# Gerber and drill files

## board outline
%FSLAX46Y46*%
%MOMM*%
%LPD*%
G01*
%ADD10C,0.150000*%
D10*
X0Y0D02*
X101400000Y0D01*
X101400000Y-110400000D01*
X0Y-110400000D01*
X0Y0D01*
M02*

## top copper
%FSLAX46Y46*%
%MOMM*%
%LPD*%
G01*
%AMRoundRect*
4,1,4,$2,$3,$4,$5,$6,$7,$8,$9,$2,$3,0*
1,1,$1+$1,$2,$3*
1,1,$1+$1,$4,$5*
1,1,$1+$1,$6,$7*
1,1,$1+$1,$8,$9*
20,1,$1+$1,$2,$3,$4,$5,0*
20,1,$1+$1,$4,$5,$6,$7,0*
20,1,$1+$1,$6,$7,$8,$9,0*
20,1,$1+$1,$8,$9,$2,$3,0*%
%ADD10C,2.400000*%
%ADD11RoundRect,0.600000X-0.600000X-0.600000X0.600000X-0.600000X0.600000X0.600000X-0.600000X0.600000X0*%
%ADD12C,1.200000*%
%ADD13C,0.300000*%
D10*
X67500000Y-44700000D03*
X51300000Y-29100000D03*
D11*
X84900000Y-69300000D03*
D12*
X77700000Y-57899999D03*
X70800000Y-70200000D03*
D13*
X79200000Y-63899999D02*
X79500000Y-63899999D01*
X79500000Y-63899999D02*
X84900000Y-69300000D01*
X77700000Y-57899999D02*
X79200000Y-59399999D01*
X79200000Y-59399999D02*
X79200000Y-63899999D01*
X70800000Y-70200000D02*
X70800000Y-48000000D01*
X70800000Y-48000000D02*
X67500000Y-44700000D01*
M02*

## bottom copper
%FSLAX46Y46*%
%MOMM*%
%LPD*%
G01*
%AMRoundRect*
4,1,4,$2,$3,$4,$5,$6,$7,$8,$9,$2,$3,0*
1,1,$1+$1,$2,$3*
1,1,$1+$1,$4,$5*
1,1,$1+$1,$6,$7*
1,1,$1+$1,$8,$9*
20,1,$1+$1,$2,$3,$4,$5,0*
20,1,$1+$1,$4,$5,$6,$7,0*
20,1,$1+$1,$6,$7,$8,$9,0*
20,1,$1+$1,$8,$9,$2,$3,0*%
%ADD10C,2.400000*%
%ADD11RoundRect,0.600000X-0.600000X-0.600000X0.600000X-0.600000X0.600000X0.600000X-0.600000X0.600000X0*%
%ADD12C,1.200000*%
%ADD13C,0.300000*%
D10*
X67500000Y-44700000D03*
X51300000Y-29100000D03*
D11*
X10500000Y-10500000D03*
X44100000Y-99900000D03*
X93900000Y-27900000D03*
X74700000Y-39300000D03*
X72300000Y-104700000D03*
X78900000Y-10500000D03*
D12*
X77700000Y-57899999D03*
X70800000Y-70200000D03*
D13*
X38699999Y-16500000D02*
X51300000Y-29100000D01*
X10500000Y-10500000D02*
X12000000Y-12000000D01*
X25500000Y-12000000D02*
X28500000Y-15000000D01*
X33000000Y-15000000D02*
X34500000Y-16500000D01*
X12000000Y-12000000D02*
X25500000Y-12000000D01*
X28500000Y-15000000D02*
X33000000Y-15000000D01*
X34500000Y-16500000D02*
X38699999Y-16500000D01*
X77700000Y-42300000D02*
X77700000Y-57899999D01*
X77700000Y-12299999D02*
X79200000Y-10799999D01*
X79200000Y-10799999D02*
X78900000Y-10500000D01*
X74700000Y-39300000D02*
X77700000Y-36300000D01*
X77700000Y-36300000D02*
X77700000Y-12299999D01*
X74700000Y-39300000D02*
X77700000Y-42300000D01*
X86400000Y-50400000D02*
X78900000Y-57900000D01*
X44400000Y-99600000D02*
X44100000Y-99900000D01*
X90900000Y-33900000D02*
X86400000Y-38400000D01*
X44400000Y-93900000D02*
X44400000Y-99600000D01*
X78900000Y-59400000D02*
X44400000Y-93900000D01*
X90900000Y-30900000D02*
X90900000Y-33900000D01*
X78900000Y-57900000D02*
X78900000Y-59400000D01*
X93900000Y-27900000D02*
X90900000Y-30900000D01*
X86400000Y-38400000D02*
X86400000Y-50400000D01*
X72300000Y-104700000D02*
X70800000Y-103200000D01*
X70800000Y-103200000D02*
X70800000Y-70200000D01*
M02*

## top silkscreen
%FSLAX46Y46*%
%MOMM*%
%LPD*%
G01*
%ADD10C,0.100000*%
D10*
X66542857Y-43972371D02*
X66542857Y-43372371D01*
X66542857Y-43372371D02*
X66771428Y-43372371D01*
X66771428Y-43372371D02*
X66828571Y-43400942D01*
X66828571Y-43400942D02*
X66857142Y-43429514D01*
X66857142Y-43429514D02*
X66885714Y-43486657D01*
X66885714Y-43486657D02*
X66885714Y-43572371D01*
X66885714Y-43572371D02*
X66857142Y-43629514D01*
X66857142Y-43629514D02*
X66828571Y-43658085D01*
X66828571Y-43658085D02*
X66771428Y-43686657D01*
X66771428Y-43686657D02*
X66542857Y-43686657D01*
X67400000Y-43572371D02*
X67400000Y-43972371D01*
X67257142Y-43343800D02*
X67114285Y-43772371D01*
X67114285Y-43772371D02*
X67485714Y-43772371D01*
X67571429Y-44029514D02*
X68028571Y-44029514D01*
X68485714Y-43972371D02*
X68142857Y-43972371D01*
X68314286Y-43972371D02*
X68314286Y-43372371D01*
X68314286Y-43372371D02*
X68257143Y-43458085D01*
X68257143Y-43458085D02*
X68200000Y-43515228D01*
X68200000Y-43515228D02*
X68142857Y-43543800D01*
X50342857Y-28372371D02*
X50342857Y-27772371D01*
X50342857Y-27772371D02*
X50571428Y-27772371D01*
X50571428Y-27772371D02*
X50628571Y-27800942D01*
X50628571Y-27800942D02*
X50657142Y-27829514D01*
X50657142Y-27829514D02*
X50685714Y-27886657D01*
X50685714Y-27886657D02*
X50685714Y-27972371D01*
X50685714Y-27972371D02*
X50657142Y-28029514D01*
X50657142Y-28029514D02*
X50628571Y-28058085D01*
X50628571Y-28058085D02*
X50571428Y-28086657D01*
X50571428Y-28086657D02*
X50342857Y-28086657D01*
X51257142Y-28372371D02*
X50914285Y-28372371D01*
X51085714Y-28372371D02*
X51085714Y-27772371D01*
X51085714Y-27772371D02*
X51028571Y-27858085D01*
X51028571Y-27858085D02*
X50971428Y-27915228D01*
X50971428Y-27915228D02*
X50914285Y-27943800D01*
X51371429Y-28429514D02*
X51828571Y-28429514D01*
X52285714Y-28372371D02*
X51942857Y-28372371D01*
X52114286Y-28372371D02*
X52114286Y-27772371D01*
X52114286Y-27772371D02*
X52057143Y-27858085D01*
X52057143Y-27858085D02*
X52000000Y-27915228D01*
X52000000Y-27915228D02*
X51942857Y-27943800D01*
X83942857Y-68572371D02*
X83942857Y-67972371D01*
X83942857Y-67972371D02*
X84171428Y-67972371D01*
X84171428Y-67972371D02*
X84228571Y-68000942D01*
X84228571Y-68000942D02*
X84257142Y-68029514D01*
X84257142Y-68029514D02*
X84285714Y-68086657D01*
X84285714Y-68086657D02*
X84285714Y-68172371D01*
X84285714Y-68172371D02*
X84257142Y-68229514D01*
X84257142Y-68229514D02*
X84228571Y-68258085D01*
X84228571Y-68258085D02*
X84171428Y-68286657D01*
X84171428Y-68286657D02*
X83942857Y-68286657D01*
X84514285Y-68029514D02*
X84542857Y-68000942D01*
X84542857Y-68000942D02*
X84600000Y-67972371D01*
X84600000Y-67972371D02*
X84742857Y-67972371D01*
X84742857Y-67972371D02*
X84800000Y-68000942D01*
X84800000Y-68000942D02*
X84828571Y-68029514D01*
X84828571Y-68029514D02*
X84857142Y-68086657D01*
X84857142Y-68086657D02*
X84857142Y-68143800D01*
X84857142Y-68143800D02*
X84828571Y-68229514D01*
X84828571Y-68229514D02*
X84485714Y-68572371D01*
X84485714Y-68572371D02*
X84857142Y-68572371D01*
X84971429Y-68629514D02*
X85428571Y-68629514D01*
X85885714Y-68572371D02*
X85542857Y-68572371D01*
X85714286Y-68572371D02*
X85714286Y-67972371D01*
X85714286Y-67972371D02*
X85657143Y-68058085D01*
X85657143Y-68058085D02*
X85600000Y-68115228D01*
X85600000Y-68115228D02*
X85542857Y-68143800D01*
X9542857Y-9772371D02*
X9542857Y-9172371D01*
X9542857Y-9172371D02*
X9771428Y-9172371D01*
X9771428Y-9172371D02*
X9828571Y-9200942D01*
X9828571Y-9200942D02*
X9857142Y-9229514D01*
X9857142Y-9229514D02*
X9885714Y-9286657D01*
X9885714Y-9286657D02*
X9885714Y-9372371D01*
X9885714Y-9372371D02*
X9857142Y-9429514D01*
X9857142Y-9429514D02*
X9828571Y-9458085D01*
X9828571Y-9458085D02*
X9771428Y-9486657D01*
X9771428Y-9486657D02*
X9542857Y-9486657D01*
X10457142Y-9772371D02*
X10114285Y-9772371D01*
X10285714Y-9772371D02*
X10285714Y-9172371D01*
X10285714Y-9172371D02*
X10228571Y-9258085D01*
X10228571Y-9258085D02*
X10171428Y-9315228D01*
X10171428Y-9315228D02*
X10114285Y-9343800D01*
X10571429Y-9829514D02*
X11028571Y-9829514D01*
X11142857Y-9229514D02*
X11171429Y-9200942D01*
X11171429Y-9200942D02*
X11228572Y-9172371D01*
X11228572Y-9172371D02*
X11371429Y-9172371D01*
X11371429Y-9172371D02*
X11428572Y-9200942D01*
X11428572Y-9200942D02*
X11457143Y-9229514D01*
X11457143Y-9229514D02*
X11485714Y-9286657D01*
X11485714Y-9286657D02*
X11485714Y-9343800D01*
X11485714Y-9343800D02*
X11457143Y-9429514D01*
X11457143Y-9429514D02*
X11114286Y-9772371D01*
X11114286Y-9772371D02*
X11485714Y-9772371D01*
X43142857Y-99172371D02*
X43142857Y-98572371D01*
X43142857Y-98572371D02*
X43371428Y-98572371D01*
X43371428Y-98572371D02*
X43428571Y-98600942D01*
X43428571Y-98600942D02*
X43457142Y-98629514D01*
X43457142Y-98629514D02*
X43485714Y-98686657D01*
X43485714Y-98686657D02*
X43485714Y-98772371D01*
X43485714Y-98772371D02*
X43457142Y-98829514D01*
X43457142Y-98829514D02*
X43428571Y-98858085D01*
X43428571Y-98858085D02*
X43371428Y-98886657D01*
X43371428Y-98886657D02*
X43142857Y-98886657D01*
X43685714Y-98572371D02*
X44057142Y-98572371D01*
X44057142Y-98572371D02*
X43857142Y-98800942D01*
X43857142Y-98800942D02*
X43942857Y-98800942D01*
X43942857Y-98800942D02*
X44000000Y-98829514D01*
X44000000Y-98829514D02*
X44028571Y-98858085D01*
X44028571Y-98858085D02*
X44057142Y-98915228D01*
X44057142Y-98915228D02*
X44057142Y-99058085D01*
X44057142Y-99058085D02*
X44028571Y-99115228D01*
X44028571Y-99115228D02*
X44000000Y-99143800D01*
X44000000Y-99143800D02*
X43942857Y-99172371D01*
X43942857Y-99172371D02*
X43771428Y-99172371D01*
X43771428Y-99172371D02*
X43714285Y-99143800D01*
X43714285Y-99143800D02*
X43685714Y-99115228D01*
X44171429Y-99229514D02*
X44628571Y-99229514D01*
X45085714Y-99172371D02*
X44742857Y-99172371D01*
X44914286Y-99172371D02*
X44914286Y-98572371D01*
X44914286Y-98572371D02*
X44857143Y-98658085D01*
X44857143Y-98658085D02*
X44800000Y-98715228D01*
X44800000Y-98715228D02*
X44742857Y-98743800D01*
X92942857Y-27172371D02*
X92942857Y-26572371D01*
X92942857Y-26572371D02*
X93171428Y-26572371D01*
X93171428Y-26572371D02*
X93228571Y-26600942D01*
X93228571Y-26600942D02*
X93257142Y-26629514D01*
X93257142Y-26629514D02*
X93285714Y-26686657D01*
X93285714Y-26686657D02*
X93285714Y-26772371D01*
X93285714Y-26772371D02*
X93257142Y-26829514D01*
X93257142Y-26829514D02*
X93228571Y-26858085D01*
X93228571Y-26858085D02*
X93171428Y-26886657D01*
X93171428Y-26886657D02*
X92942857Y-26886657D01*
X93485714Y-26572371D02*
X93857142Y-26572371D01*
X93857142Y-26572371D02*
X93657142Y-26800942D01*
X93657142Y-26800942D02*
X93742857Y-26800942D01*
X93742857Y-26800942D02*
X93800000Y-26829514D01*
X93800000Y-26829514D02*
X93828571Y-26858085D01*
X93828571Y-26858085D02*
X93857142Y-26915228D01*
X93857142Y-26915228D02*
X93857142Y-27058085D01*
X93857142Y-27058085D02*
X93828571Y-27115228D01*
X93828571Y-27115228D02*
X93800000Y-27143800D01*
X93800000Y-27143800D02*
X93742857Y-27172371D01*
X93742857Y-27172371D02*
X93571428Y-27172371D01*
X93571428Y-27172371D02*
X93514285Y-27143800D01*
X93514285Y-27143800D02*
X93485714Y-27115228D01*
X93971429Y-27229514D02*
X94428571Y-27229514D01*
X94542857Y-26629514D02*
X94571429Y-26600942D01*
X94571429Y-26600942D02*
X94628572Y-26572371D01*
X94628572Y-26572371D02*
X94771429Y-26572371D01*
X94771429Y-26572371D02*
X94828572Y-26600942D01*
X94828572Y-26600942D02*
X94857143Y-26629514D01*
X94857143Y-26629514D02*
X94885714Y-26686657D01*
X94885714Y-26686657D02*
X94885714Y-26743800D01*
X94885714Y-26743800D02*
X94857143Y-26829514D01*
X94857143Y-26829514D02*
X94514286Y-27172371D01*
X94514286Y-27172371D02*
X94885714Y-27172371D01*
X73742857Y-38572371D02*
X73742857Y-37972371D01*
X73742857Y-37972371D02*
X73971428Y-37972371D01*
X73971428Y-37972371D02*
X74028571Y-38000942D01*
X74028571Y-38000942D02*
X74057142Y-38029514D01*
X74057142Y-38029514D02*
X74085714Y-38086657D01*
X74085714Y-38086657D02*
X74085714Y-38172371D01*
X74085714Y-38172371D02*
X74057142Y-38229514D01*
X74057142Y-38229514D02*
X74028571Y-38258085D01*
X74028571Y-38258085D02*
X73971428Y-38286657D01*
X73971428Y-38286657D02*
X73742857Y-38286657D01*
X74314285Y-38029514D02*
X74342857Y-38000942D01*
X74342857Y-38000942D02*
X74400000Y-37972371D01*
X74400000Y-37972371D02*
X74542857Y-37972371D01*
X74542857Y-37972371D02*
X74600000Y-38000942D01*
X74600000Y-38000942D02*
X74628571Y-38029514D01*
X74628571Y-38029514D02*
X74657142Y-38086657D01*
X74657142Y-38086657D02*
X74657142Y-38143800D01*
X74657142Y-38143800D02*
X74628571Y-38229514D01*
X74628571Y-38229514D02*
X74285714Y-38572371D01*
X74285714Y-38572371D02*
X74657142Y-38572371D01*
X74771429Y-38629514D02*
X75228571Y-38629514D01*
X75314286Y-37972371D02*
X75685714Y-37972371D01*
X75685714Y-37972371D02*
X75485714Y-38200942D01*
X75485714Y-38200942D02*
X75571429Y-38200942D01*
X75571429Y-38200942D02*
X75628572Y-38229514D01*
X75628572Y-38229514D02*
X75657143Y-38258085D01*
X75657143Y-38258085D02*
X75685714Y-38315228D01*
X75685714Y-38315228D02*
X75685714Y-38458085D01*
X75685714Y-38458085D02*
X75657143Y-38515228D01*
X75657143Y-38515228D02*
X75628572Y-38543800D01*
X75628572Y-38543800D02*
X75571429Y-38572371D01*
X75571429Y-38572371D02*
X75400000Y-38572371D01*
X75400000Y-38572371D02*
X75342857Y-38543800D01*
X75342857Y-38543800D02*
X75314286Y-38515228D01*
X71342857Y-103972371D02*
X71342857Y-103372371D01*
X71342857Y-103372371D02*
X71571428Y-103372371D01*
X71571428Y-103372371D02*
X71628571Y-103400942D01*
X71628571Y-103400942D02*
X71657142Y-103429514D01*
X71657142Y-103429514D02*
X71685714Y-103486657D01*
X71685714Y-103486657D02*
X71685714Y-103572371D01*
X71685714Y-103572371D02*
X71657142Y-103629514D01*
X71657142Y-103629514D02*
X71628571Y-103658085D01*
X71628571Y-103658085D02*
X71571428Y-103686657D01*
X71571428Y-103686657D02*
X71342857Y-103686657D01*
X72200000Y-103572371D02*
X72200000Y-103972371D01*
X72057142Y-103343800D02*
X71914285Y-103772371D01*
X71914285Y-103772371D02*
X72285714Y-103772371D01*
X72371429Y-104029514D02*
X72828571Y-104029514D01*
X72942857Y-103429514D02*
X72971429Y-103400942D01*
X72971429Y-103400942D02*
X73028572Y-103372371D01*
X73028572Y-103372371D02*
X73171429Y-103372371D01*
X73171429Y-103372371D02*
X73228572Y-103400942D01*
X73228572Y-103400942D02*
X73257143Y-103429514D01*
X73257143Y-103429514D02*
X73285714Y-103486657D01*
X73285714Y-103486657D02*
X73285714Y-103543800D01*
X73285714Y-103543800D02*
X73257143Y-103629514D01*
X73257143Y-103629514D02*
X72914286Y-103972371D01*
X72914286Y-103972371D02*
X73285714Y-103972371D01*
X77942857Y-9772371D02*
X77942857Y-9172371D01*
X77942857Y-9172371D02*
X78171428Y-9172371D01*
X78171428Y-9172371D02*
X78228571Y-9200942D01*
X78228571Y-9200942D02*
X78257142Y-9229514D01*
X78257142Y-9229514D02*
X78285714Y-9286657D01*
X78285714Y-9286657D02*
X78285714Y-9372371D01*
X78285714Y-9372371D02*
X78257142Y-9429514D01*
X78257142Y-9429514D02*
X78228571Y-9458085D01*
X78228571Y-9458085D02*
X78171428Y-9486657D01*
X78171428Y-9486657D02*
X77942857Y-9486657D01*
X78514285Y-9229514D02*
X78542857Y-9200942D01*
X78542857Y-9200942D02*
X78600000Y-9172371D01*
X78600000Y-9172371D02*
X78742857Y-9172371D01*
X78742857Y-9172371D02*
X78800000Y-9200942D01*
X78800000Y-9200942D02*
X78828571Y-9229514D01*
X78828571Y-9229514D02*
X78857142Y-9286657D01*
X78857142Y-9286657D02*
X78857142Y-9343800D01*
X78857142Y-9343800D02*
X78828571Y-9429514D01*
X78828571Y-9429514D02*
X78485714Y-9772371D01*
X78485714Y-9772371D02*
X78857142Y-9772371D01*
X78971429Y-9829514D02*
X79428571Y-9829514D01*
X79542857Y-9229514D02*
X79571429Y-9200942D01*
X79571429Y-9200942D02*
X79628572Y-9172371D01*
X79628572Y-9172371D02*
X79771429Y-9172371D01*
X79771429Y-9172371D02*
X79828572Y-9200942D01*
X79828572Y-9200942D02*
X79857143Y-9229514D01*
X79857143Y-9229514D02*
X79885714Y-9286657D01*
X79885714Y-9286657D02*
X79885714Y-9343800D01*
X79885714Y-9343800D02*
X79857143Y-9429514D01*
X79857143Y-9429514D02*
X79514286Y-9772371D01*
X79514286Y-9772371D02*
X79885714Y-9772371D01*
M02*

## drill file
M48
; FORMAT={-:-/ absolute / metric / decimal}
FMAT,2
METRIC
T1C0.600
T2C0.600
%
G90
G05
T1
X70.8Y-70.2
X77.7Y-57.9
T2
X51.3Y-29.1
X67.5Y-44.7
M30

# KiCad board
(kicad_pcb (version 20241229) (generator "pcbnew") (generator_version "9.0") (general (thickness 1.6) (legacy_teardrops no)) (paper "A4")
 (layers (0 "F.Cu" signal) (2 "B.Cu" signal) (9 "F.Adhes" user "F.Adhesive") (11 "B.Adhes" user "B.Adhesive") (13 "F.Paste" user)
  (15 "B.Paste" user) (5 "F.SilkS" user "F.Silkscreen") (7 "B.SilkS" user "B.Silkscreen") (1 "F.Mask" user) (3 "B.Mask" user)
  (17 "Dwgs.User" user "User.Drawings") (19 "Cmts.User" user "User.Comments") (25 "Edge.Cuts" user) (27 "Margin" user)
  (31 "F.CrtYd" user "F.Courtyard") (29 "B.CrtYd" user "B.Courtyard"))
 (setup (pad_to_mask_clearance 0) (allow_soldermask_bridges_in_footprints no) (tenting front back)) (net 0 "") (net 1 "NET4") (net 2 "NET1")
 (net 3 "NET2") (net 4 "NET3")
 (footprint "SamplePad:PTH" (layer "F.Cu") (at 67.5 44.7)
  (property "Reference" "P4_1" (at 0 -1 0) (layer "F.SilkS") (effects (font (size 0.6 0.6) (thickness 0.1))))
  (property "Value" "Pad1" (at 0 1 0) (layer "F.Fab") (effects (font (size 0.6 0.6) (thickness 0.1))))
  (pad "1" thru_hole circle (at 0 0) (size 2.4 2.4) (drill 0.6) (layers "*.Cu" "*.Mask") (remove_unused_layers no) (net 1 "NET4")))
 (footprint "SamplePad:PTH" (layer "F.Cu") (at 51.3 29.1)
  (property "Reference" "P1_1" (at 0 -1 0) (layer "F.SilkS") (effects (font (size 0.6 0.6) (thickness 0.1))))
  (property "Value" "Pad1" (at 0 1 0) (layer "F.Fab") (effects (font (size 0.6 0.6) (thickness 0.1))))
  (pad "1" thru_hole circle (at 0 0) (size 2.4 2.4) (drill 0.6) (layers "*.Cu" "*.Mask") (remove_unused_layers no) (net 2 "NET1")))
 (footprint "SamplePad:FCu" (layer "F.Cu") (at 84.9 69.3)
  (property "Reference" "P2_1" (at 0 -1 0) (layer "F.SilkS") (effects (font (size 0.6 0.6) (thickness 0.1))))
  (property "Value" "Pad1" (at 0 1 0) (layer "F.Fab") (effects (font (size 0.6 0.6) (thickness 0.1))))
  (pad "1" smd roundrect (at 0 0) (size 2.4 2.4) (layers "F.Cu" "F.Mask" "F.Paste") (roundrect_rratio 0.25) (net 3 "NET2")))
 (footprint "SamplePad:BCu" (layer "B.Cu") (at 10.5 10.5)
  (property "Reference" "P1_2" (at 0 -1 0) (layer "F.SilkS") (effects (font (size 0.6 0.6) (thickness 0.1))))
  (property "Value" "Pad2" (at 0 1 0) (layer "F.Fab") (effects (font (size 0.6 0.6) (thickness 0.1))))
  (pad "1" smd roundrect (at 0 0) (size 2.4 2.4) (layers "B.Cu" "B.Mask" "B.Paste") (roundrect_rratio 0.25) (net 2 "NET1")))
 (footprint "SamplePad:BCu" (layer "B.Cu") (at 44.1 99.9)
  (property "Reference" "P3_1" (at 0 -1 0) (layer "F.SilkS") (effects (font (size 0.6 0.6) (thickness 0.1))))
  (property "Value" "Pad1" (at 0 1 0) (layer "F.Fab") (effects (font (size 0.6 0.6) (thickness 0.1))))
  (pad "1" smd roundrect (at 0 0) (size 2.4 2.4) (layers "B.Cu" "B.Mask" "B.Paste") (roundrect_rratio 0.25) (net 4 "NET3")))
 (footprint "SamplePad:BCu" (layer "B.Cu") (at 93.9 27.9)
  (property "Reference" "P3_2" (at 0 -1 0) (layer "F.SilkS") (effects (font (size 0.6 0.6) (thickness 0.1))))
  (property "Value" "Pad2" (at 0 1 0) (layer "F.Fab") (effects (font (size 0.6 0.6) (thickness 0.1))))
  (pad "1" smd roundrect (at 0 0) (size 2.4 2.4) (layers "B.Cu" "B.Mask" "B.Paste") (roundrect_rratio 0.25) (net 4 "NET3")))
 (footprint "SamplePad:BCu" (layer "B.Cu") (at 74.7 39.3)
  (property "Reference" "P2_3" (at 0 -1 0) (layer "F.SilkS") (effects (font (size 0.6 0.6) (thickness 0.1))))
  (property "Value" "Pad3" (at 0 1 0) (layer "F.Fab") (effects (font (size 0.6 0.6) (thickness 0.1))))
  (pad "1" smd roundrect (at 0 0) (size 2.4 2.4) (layers "B.Cu" "B.Mask" "B.Paste") (roundrect_rratio 0.25) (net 3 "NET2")))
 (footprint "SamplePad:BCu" (layer "B.Cu") (at 72.3 104.7)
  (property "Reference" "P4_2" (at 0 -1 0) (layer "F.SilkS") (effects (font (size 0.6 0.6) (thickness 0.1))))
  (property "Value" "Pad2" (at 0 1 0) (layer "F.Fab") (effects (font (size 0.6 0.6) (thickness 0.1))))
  (pad "1" smd roundrect (at 0 0) (size 2.4 2.4) (layers "B.Cu" "B.Mask" "B.Paste") (roundrect_rratio 0.25) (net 1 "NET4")))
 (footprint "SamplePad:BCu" (layer "B.Cu") (at 78.9 10.5)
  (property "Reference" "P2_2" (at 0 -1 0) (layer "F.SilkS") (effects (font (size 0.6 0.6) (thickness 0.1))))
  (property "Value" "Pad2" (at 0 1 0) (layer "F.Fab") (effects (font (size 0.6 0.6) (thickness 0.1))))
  (pad "1" smd roundrect (at 0 0) (size 2.4 2.4) (layers "B.Cu" "B.Mask" "B.Paste") (roundrect_rratio 0.25) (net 3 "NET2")))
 (gr_rect (start 0 0) (end 101.4 110.4) (stroke (width 0.15) (type solid)) (fill no) (layer "Edge.Cuts"))
 (segment (start 38.699999 16.5) (end 51.3 29.1) (width 0.3) (layer "B.Cu") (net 2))
 (segment (start 10.5 10.5) (end 12 12) (width 0.3) (layer "B.Cu") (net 2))
 (segment (start 25.5 12) (end 28.5 15) (width 0.3) (layer "B.Cu") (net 2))
 (segment (start 33 15) (end 34.5 16.5) (width 0.3) (layer "B.Cu") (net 2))
 (segment (start 12 12) (end 25.5 12) (width 0.3) (layer "B.Cu") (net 2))
 (segment (start 28.5 15) (end 33 15) (width 0.3) (layer "B.Cu") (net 2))
 (segment (start 34.5 16.5) (end 38.699999 16.5) (width 0.3) (layer "B.Cu") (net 2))
 (segment (start 79.2 63.899999) (end 79.5 63.899999) (width 0.3) (layer "F.Cu") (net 3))
 (segment (start 79.5 63.899999) (end 84.9 69.3) (width 0.3) (layer "F.Cu") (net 3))
 (segment (start 77.7 57.899999) (end 79.2 59.399999) (width 0.3) (layer "F.Cu") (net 3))
 (segment (start 79.2 59.399999) (end 79.2 63.899999) (width 0.3) (layer "F.Cu") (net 3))
 (via (at 77.7 57.899999) (size 1.2) (drill 0.6) (layers "F.Cu" "B.Cu") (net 3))
 (segment (start 77.7 42.3) (end 77.7 57.899999) (width 0.3) (layer "B.Cu") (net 3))
 (segment (start 77.7 12.299999) (end 79.2 10.799999) (width 0.3) (layer "B.Cu") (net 3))
 (segment (start 79.2 10.799999) (end 78.9 10.5) (width 0.3) (layer "B.Cu") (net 3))
 (segment (start 74.7 39.3) (end 77.7 36.3) (width 0.3) (layer "B.Cu") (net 3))
 (segment (start 77.7 36.3) (end 77.7 12.299999) (width 0.3) (layer "B.Cu") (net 3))
 (segment (start 74.7 39.3) (end 77.7 42.3) (width 0.3) (layer "B.Cu") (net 3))
 (segment (start 86.4 50.4) (end 78.9 57.9) (width 0.3) (layer "B.Cu") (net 4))
 (segment (start 44.4 99.6) (end 44.1 99.9) (width 0.3) (layer "B.Cu") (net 4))
 (segment (start 90.9 33.9) (end 86.4 38.4) (width 0.3) (layer "B.Cu") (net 4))
 (segment (start 44.4 93.9) (end 44.4 99.6) (width 0.3) (layer "B.Cu") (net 4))
 (segment (start 78.9 59.4) (end 44.4 93.9) (width 0.3) (layer "B.Cu") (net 4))
 (segment (start 90.9 30.9) (end 90.9 33.9) (width 0.3) (layer "B.Cu") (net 4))
 (segment (start 78.9 57.9) (end 78.9 59.4) (width 0.3) (layer "B.Cu") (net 4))
 (segment (start 93.9 27.9) (end 90.9 30.9) (width 0.3) (layer "B.Cu") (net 4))
 (segment (start 86.4 38.4) (end 86.4 50.4) (width 0.3) (layer "B.Cu") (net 4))
 (segment (start 70.8 70.2) (end 70.8 48) (width 0.3) (layer "F.Cu") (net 1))
 (segment (start 70.8 48) (end 67.5 44.7) (width 0.3) (layer "F.Cu") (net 1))
 (via (at 70.8 70.2) (size 1.2) (drill 0.6) (layers "F.Cu" "B.Cu") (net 1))
 (segment (start 72.3 104.7) (end 70.8 103.2) (width 0.3) (layer "B.Cu") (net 1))
 (segment (start 70.8 103.2) (end 70.8 70.2) (width 0.3) (layer "B.Cu") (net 1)))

